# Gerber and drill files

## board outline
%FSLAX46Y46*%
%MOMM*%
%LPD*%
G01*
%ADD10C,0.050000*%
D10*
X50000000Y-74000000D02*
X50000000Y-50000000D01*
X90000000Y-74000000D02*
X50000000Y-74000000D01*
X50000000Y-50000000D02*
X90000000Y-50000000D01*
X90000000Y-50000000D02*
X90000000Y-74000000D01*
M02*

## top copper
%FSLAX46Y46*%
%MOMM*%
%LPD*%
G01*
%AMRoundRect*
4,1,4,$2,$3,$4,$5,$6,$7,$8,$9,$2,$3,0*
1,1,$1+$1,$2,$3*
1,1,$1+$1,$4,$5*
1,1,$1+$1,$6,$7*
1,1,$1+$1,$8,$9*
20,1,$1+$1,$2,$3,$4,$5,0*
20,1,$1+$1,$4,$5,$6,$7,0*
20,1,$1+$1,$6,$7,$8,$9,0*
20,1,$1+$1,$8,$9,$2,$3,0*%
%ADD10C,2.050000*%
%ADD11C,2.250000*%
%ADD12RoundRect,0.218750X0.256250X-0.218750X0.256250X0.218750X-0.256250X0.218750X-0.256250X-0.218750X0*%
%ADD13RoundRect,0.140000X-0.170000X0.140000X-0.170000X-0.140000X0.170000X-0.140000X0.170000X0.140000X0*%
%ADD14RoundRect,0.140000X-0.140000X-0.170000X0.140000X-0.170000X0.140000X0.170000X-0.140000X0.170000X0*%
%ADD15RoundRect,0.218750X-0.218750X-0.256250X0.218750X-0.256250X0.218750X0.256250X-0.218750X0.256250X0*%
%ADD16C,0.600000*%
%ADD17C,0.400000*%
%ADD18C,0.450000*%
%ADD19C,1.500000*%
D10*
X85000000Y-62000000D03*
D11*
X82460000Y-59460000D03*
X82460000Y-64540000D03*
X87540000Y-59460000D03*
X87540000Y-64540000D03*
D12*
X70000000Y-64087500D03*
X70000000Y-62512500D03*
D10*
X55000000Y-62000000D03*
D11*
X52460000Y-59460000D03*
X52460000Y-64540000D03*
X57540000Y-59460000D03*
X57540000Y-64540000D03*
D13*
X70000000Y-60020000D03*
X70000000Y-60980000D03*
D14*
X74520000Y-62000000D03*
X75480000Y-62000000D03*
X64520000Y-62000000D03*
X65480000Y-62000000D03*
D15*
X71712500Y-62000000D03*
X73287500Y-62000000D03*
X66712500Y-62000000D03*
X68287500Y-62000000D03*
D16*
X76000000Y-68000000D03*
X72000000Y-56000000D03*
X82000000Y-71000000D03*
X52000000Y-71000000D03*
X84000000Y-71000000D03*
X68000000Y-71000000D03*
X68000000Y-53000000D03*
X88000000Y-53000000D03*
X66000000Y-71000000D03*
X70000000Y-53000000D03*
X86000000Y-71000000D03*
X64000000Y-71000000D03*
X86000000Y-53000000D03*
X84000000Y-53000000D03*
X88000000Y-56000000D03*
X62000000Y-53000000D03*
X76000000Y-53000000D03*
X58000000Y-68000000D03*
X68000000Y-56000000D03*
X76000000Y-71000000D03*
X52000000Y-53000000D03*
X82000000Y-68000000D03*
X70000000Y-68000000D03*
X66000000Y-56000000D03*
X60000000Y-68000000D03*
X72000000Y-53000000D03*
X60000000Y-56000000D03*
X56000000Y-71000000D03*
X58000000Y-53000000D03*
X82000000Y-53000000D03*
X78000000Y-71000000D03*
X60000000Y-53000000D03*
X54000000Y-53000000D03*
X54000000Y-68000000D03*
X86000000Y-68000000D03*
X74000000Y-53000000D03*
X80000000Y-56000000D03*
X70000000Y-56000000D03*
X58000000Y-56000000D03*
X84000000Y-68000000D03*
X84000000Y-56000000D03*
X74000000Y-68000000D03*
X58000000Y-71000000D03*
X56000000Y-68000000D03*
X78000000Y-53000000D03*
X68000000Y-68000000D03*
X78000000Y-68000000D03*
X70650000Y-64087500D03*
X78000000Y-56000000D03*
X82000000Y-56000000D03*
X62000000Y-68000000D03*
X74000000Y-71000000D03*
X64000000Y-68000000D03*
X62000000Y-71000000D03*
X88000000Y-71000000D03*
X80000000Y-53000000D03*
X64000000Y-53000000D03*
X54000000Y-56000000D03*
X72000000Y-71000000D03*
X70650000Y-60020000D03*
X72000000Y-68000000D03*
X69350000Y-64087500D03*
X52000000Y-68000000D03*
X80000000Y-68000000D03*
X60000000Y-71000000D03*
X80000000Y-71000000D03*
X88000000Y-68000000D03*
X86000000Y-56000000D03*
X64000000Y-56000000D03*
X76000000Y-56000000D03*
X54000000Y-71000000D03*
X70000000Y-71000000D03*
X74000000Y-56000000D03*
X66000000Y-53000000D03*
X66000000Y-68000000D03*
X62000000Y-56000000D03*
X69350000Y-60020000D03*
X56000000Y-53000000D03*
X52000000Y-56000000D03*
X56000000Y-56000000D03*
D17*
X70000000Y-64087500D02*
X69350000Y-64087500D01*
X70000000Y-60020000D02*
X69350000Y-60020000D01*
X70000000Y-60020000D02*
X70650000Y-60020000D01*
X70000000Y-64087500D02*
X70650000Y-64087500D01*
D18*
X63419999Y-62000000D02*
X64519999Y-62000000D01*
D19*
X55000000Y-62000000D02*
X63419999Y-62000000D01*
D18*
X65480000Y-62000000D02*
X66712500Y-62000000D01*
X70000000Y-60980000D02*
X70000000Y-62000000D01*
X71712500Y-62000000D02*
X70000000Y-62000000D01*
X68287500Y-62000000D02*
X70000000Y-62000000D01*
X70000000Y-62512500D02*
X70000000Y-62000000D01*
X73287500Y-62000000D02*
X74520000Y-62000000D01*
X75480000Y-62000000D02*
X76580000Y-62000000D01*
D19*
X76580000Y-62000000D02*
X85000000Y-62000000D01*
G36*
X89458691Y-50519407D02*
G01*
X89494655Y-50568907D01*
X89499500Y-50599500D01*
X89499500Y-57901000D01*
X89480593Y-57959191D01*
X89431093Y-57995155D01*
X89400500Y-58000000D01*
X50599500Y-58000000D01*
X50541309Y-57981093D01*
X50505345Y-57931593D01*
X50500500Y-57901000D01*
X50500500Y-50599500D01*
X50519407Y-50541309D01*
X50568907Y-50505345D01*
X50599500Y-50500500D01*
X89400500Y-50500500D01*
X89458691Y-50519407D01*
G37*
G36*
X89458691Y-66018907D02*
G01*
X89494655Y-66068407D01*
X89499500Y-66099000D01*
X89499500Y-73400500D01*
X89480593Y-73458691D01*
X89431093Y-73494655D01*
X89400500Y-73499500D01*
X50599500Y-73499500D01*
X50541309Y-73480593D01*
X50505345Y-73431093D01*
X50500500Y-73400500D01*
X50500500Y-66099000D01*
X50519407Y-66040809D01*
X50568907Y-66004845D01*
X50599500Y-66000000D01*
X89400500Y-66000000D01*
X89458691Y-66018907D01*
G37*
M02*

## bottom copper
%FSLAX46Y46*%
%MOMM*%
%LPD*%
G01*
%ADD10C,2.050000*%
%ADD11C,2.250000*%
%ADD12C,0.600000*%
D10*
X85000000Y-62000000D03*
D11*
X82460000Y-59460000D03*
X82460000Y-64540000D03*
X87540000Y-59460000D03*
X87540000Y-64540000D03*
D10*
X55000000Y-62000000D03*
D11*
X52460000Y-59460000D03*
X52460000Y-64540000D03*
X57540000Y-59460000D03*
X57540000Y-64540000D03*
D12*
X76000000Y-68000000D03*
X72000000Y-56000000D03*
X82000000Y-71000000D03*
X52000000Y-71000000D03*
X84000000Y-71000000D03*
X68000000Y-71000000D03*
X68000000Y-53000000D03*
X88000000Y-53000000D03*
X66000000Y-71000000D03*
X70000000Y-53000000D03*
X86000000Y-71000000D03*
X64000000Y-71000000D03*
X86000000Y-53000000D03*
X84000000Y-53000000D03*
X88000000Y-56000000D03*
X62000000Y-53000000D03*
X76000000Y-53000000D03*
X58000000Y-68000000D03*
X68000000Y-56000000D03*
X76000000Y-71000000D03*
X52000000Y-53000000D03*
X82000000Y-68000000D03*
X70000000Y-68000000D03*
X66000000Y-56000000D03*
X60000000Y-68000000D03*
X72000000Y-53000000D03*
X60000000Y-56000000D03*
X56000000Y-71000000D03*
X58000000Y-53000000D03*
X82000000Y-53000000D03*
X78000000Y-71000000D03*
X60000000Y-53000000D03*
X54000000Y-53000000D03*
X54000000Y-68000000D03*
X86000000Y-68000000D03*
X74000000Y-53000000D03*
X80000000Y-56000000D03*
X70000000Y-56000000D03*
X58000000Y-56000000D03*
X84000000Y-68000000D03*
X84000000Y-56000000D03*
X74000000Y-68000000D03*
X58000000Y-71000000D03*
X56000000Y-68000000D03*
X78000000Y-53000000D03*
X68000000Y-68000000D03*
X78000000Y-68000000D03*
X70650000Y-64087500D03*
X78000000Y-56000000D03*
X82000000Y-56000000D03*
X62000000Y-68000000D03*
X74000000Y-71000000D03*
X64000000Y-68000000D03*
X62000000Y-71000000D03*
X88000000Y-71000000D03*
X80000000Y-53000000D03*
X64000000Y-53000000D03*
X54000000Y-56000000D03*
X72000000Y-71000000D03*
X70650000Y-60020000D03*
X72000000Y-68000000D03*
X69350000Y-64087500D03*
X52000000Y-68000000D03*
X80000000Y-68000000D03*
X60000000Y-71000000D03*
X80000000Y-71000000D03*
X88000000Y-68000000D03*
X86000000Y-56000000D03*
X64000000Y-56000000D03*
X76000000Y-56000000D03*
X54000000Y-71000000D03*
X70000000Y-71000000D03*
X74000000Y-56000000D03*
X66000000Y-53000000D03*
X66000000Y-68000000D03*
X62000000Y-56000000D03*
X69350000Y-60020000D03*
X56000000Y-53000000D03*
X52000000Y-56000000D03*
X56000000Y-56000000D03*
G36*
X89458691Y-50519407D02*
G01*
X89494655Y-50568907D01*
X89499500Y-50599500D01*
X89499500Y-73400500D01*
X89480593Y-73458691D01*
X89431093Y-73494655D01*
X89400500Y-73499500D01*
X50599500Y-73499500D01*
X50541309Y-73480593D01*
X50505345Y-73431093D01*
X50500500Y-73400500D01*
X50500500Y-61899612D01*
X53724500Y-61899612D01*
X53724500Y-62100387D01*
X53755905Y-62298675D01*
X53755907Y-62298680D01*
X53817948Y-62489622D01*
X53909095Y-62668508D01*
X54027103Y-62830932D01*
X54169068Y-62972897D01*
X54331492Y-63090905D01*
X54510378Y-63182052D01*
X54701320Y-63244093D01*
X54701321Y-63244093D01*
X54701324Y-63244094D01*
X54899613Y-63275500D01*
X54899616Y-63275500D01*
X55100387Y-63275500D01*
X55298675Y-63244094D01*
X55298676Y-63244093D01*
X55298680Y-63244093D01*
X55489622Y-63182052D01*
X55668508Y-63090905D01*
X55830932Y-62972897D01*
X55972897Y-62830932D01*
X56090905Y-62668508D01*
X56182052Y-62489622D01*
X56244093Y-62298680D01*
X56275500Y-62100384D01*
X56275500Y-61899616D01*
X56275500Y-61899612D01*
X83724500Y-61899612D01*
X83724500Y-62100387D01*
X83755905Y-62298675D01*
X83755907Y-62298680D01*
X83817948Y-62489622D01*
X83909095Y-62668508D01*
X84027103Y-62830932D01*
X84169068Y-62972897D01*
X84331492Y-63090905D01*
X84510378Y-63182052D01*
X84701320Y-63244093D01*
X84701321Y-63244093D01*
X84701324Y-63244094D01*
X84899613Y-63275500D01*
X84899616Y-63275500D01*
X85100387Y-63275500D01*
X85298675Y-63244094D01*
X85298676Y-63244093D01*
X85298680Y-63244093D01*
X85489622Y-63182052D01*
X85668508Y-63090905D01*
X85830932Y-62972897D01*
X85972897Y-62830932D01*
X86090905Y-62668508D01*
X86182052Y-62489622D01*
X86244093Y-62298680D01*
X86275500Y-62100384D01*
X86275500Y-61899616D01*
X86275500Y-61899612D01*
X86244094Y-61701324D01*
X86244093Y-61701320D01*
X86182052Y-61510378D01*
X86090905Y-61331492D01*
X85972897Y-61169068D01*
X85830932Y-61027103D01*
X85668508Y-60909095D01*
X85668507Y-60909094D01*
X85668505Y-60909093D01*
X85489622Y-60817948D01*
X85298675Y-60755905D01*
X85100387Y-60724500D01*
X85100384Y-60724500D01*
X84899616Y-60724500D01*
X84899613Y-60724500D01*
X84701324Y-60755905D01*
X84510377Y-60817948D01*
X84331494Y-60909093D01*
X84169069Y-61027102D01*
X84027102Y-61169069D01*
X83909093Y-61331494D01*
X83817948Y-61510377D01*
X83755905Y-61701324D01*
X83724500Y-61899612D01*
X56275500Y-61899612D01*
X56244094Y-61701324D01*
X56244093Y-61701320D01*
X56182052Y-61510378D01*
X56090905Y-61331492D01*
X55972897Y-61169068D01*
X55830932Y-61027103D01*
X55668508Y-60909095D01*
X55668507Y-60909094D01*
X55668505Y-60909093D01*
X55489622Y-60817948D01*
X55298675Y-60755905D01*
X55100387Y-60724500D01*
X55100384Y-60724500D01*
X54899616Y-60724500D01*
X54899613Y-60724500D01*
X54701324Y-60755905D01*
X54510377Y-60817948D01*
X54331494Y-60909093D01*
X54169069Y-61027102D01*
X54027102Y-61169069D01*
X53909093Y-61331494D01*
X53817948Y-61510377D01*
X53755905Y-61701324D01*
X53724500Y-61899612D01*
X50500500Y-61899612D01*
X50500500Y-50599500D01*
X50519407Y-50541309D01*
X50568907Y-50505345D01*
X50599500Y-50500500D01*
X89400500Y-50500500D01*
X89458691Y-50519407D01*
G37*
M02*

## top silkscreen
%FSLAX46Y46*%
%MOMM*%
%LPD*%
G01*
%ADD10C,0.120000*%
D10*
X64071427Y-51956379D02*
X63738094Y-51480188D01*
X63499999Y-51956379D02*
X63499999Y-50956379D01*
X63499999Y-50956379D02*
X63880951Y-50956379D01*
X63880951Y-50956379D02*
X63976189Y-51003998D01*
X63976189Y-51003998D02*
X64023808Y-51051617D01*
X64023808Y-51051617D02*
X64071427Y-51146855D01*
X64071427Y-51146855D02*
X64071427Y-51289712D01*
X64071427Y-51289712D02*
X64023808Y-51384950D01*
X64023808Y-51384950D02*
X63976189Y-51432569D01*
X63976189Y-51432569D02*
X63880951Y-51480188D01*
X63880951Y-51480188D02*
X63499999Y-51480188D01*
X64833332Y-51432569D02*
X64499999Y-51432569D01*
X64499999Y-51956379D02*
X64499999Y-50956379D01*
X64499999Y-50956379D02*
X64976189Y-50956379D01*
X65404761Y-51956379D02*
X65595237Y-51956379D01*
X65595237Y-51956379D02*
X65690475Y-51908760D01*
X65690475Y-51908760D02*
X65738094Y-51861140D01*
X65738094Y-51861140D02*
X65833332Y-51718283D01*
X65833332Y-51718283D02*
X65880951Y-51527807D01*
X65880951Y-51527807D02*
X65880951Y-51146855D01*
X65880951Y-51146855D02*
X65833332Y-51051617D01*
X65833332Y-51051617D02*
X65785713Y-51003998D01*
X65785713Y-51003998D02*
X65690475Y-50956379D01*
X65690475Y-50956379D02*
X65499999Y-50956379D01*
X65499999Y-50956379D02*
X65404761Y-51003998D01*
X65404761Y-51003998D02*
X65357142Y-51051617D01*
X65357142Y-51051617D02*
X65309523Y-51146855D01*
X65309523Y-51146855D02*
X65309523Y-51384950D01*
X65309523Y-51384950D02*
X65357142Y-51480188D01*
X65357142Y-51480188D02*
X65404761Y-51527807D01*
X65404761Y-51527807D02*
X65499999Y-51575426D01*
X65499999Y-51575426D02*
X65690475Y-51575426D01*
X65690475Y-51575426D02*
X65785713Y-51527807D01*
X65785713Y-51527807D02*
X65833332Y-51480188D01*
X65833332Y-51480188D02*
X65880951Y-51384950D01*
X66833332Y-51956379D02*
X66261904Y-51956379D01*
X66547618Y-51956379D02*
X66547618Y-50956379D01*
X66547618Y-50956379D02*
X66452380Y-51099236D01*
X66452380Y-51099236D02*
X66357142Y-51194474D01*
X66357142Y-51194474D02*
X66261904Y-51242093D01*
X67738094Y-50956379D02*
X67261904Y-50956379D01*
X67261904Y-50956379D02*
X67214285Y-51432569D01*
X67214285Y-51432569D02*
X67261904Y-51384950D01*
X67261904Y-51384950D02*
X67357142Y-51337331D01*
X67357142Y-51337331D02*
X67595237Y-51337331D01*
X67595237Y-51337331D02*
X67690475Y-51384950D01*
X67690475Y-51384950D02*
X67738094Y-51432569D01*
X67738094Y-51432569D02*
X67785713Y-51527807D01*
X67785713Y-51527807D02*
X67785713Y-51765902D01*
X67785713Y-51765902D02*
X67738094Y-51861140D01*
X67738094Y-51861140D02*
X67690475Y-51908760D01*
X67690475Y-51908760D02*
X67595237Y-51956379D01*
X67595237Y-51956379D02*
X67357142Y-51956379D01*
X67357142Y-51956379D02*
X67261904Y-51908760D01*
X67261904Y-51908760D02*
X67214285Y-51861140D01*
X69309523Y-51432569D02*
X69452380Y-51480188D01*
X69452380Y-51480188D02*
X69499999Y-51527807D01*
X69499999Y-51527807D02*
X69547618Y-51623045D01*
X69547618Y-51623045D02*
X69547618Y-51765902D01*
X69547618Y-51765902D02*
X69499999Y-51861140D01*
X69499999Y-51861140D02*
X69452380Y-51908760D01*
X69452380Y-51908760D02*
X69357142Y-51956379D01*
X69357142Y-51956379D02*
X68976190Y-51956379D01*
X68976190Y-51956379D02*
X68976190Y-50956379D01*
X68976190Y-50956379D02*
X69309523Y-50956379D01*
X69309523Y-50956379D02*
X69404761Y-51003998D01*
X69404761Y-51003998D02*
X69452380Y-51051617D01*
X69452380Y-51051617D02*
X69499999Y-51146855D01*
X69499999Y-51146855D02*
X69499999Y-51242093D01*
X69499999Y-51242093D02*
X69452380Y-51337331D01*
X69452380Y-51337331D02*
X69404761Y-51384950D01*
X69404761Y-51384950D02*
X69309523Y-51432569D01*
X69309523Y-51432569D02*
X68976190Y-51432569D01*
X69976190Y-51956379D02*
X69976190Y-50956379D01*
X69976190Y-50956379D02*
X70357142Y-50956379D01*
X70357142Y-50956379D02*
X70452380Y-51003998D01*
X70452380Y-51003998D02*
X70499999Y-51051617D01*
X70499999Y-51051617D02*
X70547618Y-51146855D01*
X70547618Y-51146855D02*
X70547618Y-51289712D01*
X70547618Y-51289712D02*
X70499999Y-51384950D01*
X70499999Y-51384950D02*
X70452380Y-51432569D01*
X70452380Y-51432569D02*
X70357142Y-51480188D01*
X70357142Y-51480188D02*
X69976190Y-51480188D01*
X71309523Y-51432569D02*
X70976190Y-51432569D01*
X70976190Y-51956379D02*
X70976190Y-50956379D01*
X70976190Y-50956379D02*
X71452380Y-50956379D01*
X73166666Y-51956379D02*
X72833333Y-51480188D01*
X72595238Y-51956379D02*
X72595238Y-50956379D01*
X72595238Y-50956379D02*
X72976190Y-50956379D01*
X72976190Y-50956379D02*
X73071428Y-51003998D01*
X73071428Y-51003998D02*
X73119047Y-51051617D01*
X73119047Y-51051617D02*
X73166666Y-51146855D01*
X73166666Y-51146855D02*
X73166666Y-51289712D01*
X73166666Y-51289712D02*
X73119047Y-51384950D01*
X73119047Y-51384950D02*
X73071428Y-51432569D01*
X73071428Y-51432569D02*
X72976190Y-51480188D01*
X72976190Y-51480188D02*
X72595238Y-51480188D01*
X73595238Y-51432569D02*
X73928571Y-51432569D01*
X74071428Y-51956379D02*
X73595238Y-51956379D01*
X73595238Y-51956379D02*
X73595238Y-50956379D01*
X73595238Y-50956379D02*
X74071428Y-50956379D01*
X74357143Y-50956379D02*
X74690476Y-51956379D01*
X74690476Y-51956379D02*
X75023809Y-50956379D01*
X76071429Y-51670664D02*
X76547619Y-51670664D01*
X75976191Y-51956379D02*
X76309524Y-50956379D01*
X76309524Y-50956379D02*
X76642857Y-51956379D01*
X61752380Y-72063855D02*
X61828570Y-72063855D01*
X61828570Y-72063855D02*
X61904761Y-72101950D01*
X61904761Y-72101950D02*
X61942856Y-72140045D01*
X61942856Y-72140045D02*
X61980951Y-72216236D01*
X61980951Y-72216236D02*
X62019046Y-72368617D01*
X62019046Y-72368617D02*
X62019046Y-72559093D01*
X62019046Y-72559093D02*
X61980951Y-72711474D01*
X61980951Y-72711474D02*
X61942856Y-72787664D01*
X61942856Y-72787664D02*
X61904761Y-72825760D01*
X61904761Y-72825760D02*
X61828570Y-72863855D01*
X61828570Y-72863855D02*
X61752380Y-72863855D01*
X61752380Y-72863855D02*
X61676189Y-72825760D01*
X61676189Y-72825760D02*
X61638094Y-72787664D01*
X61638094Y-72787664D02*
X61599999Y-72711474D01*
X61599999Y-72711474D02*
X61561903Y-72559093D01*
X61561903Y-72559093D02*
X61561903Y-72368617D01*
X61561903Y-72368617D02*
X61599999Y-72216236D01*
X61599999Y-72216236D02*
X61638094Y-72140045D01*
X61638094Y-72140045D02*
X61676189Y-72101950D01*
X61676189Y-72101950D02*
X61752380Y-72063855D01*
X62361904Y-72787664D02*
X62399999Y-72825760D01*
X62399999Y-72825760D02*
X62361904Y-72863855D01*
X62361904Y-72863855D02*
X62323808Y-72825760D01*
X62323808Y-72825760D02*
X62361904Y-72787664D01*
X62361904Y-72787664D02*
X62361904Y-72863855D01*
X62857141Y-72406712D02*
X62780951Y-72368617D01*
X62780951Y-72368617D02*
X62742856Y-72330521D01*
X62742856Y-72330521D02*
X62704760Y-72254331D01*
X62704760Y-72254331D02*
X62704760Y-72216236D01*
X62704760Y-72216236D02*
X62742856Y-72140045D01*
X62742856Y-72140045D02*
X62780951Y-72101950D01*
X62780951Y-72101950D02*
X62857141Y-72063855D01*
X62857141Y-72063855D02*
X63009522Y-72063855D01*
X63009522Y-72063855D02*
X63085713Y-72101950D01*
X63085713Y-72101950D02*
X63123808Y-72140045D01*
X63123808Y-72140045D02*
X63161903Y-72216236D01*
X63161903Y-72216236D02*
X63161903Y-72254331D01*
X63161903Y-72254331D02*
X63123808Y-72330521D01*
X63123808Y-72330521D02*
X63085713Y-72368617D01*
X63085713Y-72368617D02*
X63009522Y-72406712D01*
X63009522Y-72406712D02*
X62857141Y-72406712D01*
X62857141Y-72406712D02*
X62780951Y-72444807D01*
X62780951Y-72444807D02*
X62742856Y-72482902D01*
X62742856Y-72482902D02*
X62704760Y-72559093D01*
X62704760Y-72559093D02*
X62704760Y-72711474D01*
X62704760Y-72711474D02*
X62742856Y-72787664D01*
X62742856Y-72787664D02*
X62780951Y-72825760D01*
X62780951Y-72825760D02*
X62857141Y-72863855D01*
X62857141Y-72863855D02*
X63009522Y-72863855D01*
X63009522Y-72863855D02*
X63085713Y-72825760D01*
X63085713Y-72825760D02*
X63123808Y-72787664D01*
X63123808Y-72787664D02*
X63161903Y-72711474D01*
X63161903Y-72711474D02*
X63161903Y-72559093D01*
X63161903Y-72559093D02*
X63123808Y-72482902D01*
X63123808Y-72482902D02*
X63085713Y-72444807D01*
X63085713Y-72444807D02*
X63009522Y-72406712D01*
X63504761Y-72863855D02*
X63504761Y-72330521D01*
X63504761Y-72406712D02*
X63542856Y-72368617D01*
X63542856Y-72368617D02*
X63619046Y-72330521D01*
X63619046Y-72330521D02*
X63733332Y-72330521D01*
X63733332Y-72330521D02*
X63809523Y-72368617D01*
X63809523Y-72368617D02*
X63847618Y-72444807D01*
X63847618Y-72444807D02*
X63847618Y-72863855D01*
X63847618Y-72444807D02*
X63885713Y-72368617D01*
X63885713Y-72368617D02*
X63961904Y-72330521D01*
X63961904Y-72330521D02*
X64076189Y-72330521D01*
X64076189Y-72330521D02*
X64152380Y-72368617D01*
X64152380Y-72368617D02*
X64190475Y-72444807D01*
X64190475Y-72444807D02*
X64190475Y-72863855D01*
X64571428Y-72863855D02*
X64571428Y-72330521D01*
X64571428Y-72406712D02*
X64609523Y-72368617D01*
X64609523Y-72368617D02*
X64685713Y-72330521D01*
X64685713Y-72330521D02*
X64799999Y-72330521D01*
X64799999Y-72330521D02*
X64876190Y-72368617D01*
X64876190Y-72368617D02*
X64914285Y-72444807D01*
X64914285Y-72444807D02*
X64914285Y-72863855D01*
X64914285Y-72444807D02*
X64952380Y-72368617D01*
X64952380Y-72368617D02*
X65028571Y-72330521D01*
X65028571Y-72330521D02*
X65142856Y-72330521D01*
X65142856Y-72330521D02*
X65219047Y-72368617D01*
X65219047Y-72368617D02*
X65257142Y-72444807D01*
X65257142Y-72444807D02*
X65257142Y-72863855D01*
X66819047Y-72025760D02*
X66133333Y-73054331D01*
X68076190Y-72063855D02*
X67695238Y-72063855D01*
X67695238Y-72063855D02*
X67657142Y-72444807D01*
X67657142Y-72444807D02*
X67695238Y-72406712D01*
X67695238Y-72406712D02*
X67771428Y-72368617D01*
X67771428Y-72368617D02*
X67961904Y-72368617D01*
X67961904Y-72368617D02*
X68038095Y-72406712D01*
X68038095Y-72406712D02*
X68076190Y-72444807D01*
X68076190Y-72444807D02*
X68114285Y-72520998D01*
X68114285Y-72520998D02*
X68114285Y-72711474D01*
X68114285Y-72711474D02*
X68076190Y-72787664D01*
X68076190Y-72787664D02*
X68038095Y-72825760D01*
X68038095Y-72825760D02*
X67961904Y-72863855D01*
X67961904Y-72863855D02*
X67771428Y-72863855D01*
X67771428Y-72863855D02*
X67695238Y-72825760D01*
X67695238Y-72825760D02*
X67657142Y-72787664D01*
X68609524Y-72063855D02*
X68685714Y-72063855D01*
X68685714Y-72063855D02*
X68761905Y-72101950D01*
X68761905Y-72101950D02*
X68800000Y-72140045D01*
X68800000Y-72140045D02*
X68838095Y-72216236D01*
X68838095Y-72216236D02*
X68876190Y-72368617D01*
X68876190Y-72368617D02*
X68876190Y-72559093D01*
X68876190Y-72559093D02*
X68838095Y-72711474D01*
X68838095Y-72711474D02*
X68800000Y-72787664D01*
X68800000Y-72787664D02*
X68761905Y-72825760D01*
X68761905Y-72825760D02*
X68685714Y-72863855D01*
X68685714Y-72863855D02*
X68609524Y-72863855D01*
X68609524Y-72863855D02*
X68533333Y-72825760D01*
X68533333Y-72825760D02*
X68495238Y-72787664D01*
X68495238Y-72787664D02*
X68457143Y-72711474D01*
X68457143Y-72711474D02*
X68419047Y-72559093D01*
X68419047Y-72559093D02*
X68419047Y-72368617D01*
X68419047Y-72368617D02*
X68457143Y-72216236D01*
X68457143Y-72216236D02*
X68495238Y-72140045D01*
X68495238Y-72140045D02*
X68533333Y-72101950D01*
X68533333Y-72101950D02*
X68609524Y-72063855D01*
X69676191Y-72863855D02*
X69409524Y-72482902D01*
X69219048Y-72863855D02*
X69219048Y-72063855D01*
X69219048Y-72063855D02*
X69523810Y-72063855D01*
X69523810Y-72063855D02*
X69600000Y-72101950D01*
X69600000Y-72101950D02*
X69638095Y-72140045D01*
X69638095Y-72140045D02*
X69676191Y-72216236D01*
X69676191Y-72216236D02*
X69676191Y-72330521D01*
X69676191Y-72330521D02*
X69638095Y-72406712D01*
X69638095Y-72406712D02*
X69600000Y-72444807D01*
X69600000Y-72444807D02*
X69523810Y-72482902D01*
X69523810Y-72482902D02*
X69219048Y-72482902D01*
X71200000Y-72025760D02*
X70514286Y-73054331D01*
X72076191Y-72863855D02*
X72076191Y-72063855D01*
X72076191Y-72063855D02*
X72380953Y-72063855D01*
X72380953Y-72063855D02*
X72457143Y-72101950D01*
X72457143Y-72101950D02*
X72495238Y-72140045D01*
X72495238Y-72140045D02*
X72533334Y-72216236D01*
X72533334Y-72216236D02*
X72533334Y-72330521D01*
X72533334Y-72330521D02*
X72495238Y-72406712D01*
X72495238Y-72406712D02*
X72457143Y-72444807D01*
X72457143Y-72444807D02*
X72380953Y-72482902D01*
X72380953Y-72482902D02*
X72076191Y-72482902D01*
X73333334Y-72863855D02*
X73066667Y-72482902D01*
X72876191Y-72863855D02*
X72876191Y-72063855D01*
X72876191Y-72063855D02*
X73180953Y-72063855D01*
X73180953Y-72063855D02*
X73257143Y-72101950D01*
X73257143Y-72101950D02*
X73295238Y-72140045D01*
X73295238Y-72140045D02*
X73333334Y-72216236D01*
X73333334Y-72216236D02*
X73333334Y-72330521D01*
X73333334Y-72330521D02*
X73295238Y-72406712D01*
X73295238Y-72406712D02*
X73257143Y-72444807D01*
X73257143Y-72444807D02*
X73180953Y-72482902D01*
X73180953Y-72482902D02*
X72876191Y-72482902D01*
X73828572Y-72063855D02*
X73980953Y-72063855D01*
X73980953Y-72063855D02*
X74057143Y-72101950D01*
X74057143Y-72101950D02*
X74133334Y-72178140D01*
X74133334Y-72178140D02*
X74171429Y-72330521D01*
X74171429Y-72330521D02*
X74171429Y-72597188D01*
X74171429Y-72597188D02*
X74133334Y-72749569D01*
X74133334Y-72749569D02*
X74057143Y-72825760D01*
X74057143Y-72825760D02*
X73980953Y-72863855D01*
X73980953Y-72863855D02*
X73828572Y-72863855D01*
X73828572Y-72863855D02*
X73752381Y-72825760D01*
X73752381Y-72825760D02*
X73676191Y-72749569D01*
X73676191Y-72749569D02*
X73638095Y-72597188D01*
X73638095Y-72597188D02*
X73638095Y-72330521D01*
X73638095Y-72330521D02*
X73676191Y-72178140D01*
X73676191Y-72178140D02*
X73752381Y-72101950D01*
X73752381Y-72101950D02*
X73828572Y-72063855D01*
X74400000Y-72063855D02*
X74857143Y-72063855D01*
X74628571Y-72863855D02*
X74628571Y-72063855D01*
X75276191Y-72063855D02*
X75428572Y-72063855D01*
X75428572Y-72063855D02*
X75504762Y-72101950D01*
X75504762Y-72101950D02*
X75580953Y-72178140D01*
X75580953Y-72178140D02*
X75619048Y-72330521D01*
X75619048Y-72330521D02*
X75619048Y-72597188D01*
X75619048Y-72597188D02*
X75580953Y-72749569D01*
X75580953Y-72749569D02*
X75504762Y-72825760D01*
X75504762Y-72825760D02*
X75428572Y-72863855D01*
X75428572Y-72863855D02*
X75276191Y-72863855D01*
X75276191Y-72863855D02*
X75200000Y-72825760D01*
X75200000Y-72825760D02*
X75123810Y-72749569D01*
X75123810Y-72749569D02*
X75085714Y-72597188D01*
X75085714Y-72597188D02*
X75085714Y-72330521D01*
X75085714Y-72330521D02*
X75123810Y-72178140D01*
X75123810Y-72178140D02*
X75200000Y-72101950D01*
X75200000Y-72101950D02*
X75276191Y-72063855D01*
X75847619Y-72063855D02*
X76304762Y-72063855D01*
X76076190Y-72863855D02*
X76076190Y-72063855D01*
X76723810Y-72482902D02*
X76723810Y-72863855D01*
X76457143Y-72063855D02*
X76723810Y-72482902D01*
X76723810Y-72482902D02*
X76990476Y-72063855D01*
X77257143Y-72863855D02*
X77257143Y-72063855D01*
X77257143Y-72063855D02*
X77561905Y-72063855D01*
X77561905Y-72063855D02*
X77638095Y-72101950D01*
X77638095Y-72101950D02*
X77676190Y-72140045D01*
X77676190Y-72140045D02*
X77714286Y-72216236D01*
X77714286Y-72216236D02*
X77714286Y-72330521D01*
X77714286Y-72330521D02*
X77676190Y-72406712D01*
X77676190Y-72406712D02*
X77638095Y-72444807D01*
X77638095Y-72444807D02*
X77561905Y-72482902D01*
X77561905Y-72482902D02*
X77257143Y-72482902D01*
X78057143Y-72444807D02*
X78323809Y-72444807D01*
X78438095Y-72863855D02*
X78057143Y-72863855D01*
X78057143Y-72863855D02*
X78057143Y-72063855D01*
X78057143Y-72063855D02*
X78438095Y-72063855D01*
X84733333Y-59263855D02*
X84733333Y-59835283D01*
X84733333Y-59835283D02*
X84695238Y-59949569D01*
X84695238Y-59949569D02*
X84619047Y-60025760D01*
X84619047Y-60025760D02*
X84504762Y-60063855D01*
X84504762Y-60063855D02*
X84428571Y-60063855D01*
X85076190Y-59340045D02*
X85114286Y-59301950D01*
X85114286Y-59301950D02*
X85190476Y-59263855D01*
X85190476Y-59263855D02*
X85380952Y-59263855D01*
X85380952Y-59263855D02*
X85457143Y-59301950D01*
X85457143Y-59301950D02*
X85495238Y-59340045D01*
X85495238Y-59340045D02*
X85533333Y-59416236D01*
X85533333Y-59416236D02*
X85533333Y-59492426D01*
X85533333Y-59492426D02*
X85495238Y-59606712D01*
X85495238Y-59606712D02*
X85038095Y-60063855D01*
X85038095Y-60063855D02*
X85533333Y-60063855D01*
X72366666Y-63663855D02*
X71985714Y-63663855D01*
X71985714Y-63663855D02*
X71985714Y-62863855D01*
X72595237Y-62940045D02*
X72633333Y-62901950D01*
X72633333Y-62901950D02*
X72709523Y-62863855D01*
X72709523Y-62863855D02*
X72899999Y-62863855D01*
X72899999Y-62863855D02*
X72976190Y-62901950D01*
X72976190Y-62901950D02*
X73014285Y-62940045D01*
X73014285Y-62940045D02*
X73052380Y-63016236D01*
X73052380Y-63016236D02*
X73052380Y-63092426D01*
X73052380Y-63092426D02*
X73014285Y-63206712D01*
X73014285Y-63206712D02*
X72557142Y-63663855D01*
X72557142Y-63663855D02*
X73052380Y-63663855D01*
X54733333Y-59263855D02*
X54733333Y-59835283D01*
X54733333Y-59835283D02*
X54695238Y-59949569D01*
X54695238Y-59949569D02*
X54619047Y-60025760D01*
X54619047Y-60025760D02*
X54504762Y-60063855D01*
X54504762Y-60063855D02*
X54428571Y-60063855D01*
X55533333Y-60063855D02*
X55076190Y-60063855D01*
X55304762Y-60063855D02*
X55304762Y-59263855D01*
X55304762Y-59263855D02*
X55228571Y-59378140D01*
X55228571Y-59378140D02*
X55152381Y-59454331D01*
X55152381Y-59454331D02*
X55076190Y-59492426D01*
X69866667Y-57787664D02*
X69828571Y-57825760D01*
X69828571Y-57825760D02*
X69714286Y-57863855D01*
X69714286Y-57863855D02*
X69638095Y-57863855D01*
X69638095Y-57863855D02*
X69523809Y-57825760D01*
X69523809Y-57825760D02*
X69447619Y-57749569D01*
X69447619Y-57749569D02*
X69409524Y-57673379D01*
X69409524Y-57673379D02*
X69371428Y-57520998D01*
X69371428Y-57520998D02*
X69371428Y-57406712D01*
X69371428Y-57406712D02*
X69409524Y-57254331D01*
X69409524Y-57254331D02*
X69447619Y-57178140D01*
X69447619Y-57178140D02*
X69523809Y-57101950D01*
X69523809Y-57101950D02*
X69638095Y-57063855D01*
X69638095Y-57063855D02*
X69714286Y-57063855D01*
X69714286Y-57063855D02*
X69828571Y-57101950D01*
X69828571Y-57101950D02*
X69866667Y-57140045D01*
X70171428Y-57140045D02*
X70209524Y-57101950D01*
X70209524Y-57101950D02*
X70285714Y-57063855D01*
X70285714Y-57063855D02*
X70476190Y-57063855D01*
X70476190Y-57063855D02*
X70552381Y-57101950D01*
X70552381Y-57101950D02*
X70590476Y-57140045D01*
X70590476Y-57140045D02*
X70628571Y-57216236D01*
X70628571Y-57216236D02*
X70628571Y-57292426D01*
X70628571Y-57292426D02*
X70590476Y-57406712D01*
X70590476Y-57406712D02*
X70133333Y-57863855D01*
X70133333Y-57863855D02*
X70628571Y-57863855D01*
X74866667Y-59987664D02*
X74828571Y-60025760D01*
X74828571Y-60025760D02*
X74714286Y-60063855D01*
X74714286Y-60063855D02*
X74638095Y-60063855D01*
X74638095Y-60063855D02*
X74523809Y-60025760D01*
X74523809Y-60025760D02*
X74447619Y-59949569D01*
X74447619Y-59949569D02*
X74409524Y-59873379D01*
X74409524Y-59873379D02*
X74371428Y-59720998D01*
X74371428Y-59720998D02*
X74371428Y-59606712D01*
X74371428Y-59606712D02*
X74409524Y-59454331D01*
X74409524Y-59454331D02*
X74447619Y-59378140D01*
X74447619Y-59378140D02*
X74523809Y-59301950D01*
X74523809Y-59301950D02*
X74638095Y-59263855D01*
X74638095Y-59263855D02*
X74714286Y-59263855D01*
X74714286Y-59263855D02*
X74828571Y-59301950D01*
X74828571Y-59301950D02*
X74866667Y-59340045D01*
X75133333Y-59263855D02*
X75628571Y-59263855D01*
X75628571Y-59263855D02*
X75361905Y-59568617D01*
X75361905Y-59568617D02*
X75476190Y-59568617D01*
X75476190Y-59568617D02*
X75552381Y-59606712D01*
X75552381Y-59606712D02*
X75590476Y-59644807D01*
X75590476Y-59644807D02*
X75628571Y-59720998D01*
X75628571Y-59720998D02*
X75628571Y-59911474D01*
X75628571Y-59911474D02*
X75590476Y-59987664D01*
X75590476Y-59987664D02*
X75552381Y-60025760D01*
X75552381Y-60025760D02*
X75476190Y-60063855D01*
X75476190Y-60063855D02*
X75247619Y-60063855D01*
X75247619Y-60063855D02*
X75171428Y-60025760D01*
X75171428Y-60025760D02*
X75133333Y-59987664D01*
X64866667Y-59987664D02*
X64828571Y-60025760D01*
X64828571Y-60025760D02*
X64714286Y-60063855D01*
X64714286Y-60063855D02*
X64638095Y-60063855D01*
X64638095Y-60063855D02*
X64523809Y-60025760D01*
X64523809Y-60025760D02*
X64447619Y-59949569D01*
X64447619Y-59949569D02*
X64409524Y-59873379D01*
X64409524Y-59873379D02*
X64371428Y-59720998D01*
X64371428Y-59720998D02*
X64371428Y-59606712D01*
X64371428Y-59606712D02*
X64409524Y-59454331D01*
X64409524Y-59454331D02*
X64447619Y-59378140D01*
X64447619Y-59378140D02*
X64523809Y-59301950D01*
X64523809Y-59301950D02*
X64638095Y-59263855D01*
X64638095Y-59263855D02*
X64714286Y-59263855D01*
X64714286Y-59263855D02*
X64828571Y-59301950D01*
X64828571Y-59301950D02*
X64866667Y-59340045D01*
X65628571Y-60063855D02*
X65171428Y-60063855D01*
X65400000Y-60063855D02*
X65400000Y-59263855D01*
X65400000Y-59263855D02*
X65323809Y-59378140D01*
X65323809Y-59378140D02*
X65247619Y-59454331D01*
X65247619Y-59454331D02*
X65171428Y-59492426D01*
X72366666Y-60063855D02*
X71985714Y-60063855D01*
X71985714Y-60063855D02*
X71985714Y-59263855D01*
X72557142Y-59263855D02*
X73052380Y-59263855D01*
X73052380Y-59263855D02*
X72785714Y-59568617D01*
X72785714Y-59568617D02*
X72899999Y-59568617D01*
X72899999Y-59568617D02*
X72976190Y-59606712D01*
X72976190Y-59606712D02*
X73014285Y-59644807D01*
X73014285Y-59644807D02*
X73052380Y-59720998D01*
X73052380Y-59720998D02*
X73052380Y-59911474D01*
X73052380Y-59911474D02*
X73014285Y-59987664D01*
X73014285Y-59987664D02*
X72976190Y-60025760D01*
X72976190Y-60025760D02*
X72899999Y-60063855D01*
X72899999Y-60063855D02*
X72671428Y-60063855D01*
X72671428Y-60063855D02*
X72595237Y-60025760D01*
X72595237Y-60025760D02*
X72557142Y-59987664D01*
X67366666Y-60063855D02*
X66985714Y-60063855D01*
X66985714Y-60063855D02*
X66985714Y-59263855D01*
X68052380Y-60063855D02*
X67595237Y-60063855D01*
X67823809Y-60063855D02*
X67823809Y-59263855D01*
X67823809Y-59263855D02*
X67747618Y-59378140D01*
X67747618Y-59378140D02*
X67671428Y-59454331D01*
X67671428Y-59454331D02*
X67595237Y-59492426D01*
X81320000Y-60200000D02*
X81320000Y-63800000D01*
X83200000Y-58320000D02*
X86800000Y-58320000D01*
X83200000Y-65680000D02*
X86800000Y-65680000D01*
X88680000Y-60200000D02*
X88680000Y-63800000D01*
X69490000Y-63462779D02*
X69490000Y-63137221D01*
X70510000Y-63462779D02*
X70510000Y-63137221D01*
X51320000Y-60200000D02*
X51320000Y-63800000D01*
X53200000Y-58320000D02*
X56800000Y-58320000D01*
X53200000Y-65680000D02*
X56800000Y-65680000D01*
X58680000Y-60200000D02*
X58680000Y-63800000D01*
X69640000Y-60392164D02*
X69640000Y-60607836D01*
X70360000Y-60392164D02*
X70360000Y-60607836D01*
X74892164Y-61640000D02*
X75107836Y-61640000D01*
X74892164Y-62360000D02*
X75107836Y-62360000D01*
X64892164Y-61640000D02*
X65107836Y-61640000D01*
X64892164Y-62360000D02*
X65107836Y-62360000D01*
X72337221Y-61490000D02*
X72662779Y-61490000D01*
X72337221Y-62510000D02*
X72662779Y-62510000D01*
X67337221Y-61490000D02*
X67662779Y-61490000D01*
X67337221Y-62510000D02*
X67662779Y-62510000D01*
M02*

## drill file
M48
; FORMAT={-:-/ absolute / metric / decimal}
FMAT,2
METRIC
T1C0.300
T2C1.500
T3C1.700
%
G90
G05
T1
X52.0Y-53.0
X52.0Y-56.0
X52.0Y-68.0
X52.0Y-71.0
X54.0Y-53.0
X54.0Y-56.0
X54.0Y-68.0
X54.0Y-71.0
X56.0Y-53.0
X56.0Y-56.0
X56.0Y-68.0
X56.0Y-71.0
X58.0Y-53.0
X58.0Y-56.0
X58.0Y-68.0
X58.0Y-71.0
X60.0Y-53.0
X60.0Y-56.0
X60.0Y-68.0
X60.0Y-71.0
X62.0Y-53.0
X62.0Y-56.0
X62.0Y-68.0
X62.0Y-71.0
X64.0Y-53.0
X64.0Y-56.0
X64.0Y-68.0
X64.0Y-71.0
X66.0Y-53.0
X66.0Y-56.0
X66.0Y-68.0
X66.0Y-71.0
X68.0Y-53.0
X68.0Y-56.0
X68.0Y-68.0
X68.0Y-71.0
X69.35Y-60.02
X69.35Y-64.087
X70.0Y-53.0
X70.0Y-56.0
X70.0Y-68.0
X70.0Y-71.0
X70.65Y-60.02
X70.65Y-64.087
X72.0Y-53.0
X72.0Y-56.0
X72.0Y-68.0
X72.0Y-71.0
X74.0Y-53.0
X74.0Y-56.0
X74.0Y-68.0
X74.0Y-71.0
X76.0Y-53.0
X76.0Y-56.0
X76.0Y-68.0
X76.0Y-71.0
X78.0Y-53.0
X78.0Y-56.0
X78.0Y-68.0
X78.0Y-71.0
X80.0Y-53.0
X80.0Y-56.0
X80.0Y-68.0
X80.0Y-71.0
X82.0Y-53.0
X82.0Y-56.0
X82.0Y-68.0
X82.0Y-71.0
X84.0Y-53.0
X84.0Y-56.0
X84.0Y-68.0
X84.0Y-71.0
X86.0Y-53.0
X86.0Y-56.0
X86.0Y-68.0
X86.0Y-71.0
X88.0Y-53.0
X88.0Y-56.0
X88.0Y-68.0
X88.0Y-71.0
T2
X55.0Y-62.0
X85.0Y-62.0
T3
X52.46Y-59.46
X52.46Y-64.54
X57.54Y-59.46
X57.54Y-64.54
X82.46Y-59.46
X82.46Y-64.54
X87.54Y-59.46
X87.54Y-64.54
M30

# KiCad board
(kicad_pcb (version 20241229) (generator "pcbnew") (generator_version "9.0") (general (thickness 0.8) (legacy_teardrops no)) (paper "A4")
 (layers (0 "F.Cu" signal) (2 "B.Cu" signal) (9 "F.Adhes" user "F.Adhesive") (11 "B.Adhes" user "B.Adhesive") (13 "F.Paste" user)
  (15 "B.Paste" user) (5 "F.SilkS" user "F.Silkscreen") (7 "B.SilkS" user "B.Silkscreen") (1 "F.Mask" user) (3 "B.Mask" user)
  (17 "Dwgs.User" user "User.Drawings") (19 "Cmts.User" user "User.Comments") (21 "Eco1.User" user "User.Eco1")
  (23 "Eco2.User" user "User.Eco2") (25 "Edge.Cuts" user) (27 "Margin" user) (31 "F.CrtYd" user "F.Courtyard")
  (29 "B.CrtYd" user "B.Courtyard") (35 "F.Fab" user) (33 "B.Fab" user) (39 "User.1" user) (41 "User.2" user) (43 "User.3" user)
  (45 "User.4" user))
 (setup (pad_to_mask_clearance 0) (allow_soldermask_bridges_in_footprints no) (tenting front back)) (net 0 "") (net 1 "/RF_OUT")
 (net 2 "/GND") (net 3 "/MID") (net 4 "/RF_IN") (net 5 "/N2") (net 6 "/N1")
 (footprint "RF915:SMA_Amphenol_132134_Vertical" (layer "F.Cu") (at 85 62)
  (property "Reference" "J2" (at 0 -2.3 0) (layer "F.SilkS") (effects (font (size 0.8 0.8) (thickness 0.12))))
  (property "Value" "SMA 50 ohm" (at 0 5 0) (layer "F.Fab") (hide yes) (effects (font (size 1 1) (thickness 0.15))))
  (fp_line (start -3.68 -1.8) (end -3.68 1.8) (stroke (width 0.12) (type solid)) (layer "F.SilkS"))
  (fp_line (start -1.8 -3.68) (end 1.8 -3.68) (stroke (width 0.12) (type solid)) (layer "F.SilkS"))
  (fp_line (start -1.8 3.68) (end 1.8 3.68) (stroke (width 0.12) (type solid)) (layer "F.SilkS"))
  (fp_line (start 3.68 -1.8) (end 3.68 1.8) (stroke (width 0.12) (type solid)) (layer "F.SilkS"))
  (pad "1" thru_hole circle (at 0 0) (size 2.05 2.05) (drill 1.5) (layers "*.Cu" "*.Mask") (remove_unused_layers no) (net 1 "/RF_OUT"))
  (pad "2" thru_hole circle (at -2.54 -2.54) (size 2.25 2.25) (drill 1.7) (layers "*.Cu" "*.Mask") (remove_unused_layers no) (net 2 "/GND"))
  (pad "2" thru_hole circle (at -2.54 2.54) (size 2.25 2.25) (drill 1.7) (layers "*.Cu" "*.Mask") (remove_unused_layers no) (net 2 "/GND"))
  (pad "2" thru_hole circle (at 2.54 -2.54) (size 2.25 2.25) (drill 1.7) (layers "*.Cu" "*.Mask") (remove_unused_layers no) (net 2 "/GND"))
  (pad "2" thru_hole circle (at 2.54 2.54) (size 2.25 2.25) (drill 1.7) (layers "*.Cu" "*.Mask") (remove_unused_layers no) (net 2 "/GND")))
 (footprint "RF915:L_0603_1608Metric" (layer "F.Cu") (at 70 63.3 90)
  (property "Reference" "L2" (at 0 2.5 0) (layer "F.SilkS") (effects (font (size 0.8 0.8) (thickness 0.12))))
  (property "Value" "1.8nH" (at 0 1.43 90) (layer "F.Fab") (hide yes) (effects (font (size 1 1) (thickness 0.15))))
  (fp_line (start -0.162779 -0.51) (end 0.162779 -0.51) (stroke (width 0.12) (type solid)) (layer "F.SilkS"))
  (fp_line (start -0.162779 0.51) (end 0.162779 0.51) (stroke (width 0.12) (type solid)) (layer "F.SilkS"))
  (pad "1" smd roundrect (at -0.7875 0 90) (size 0.875 0.95) (layers "F.Cu" "F.Mask" "F.Paste") (roundrect_rratio 0.25) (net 2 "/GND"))
  (pad "2" smd roundrect (at 0.7875 0 90) (size 0.875 0.95) (layers "F.Cu" "F.Mask" "F.Paste") (roundrect_rratio 0.25) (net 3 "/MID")))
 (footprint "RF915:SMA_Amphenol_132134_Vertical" (layer "F.Cu") (at 55 62)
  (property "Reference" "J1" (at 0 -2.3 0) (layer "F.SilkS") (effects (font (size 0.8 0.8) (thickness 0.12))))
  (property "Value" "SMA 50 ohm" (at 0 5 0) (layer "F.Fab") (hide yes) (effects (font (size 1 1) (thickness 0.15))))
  (fp_line (start -3.68 -1.8) (end -3.68 1.8) (stroke (width 0.12) (type solid)) (layer "F.SilkS"))
  (fp_line (start -1.8 -3.68) (end 1.8 -3.68) (stroke (width 0.12) (type solid)) (layer "F.SilkS"))
  (fp_line (start -1.8 3.68) (end 1.8 3.68) (stroke (width 0.12) (type solid)) (layer "F.SilkS"))
  (fp_line (start 3.68 -1.8) (end 3.68 1.8) (stroke (width 0.12) (type solid)) (layer "F.SilkS"))
  (pad "1" thru_hole circle (at 0 0) (size 2.05 2.05) (drill 1.5) (layers "*.Cu" "*.Mask") (remove_unused_layers no) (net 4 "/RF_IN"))
  (pad "2" thru_hole circle (at -2.54 -2.54) (size 2.25 2.25) (drill 1.7) (layers "*.Cu" "*.Mask") (remove_unused_layers no) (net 2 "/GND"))
  (pad "2" thru_hole circle (at -2.54 2.54) (size 2.25 2.25) (drill 1.7) (layers "*.Cu" "*.Mask") (remove_unused_layers no) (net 2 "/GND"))
  (pad "2" thru_hole circle (at 2.54 -2.54) (size 2.25 2.25) (drill 1.7) (layers "*.Cu" "*.Mask") (remove_unused_layers no) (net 2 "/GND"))
  (pad "2" thru_hole circle (at 2.54 2.54) (size 2.25 2.25) (drill 1.7) (layers "*.Cu" "*.Mask") (remove_unused_layers no) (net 2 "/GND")))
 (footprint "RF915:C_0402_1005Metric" (layer "F.Cu") (at 70 60.5 -90)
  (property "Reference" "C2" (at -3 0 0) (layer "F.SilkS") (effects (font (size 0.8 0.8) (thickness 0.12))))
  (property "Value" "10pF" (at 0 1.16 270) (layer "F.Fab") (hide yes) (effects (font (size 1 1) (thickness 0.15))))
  (fp_line (start -0.107836 0.36) (end 0.107836 0.36) (stroke (width 0.12) (type solid)) (layer "F.SilkS"))
  (fp_line (start -0.107836 -0.36) (end 0.107836 -0.36) (stroke (width 0.12) (type solid)) (layer "F.SilkS"))
  (pad "1" smd roundrect (at -0.48 0 270) (size 0.56 0.62) (layers "F.Cu" "F.Mask" "F.Paste") (roundrect_rratio 0.25) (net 2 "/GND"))
  (pad "2" smd roundrect (at 0.48 0 270) (size 0.56 0.62) (layers "F.Cu" "F.Mask" "F.Paste") (roundrect_rratio 0.25) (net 3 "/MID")))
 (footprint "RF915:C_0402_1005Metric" (layer "F.Cu") (at 75 62)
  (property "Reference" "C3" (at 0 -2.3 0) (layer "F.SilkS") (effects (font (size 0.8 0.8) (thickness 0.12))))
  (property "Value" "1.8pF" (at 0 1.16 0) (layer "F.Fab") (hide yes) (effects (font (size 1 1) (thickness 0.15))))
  (fp_line (start -0.107836 -0.36) (end 0.107836 -0.36) (stroke (width 0.12) (type solid)) (layer "F.SilkS"))
  (fp_line (start -0.107836 0.36) (end 0.107836 0.36) (stroke (width 0.12) (type solid)) (layer "F.SilkS"))
  (pad "1" smd roundrect (at -0.48 0) (size 0.56 0.62) (layers "F.Cu" "F.Mask" "F.Paste") (roundrect_rratio 0.25) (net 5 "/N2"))
  (pad "2" smd roundrect (at 0.48 0) (size 0.56 0.62) (layers "F.Cu" "F.Mask" "F.Paste") (roundrect_rratio 0.25) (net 1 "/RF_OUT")))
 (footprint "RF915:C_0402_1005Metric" (layer "F.Cu") (at 65 62)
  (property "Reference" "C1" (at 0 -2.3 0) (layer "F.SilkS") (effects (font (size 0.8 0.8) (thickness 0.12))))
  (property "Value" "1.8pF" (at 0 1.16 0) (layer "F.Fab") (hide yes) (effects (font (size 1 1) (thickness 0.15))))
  (fp_line (start -0.107836 -0.36) (end 0.107836 -0.36) (stroke (width 0.12) (type solid)) (layer "F.SilkS"))
  (fp_line (start -0.107836 0.36) (end 0.107836 0.36) (stroke (width 0.12) (type solid)) (layer "F.SilkS"))
  (pad "1" smd roundrect (at -0.48 0) (size 0.56 0.62) (layers "F.Cu" "F.Mask" "F.Paste") (roundrect_rratio 0.25) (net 4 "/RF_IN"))
  (pad "2" smd roundrect (at 0.48 0) (size 0.56 0.62) (layers "F.Cu" "F.Mask" "F.Paste") (roundrect_rratio 0.25) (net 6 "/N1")))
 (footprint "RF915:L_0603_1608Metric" (layer "F.Cu") (at 72.5 62)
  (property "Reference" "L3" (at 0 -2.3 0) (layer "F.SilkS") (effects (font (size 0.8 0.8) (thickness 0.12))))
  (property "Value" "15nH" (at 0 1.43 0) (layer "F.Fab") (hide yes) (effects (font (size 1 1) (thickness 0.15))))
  (fp_line (start -0.162779 -0.51) (end 0.162779 -0.51) (stroke (width 0.12) (type solid)) (layer "F.SilkS"))
  (fp_line (start -0.162779 0.51) (end 0.162779 0.51) (stroke (width 0.12) (type solid)) (layer "F.SilkS"))
  (pad "1" smd roundrect (at -0.7875 0) (size 0.875 0.95) (layers "F.Cu" "F.Mask" "F.Paste") (roundrect_rratio 0.25) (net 3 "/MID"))
  (pad "2" smd roundrect (at 0.7875 0) (size 0.875 0.95) (layers "F.Cu" "F.Mask" "F.Paste") (roundrect_rratio 0.25) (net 5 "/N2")))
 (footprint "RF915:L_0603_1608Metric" (layer "F.Cu") (at 67.5 62)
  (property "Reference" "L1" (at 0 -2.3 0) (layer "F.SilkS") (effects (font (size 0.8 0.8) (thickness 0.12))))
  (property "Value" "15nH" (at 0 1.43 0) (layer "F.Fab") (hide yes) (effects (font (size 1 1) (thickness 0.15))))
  (fp_line (start -0.162779 -0.51) (end 0.162779 -0.51) (stroke (width 0.12) (type solid)) (layer "F.SilkS"))
  (fp_line (start -0.162779 0.51) (end 0.162779 0.51) (stroke (width 0.12) (type solid)) (layer "F.SilkS"))
  (pad "1" smd roundrect (at -0.7875 0) (size 0.875 0.95) (layers "F.Cu" "F.Mask" "F.Paste") (roundrect_rratio 0.25) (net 6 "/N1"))
  (pad "2" smd roundrect (at 0.7875 0) (size 0.875 0.95) (layers "F.Cu" "F.Mask" "F.Paste") (roundrect_rratio 0.25) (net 3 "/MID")))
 (gr_line (start 50 74) (end 50 50) (stroke (width 0.05) (type default)) (layer "Edge.Cuts"))
 (gr_line (start 90 74) (end 50 74) (stroke (width 0.05) (type default)) (layer "Edge.Cuts"))
 (gr_line (start 50 50) (end 90 50) (stroke (width 0.05) (type default)) (layer "Edge.Cuts"))
 (gr_line (start 90 50) (end 90 74) (stroke (width 0.05) (type default)) (layer "Edge.Cuts"))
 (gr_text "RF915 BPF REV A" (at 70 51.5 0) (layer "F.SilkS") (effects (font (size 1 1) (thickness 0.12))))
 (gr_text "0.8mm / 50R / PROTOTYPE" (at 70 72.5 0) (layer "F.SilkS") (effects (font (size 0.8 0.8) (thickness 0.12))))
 (segment (start 70 64.0875) (end 69.35 64.0875) (width 0.4) (layer "F.Cu") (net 2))
 (segment (start 70 60.02) (end 69.35 60.02) (width 0.4) (layer "F.Cu") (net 2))
 (segment (start 70 60.02) (end 70.65 60.02) (width 0.4) (layer "F.Cu") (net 2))
 (segment (start 70 64.0875) (end 70.65 64.0875) (width 0.4) (layer "F.Cu") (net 2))
 (via (at 76 68) (size 0.6) (drill 0.3) (layers "F.Cu" "B.Cu") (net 2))
 (via (at 72 56) (size 0.6) (drill 0.3) (layers "F.Cu" "B.Cu") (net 2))
 (via (at 82 71) (size 0.6) (drill 0.3) (layers "F.Cu" "B.Cu") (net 2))
 (via (at 52 71) (size 0.6) (drill 0.3) (layers "F.Cu" "B.Cu") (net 2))
 (via (at 84 71) (size 0.6) (drill 0.3) (layers "F.Cu" "B.Cu") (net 2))
 (via (at 68 71) (size 0.6) (drill 0.3) (layers "F.Cu" "B.Cu") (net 2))
 (via (at 68 53) (size 0.6) (drill 0.3) (layers "F.Cu" "B.Cu") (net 2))
 (via (at 88 53) (size 0.6) (drill 0.3) (layers "F.Cu" "B.Cu") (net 2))
 (via (at 66 71) (size 0.6) (drill 0.3) (layers "F.Cu" "B.Cu") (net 2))
 (via (at 70 53) (size 0.6) (drill 0.3) (layers "F.Cu" "B.Cu") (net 2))
 (via (at 86 71) (size 0.6) (drill 0.3) (layers "F.Cu" "B.Cu") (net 2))
 (via (at 64 71) (size 0.6) (drill 0.3) (layers "F.Cu" "B.Cu") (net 2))
 (via (at 86 53) (size 0.6) (drill 0.3) (layers "F.Cu" "B.Cu") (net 2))
 (via (at 84 53) (size 0.6) (drill 0.3) (layers "F.Cu" "B.Cu") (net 2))
 (via (at 88 56) (size 0.6) (drill 0.3) (layers "F.Cu" "B.Cu") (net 2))
 (via (at 62 53) (size 0.6) (drill 0.3) (layers "F.Cu" "B.Cu") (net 2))
 (via (at 76 53) (size 0.6) (drill 0.3) (layers "F.Cu" "B.Cu") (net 2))
 (via (at 58 68) (size 0.6) (drill 0.3) (layers "F.Cu" "B.Cu") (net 2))
 (via (at 68 56) (size 0.6) (drill 0.3) (layers "F.Cu" "B.Cu") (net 2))
 (via (at 76 71) (size 0.6) (drill 0.3) (layers "F.Cu" "B.Cu") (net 2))
 (via (at 52 53) (size 0.6) (drill 0.3) (layers "F.Cu" "B.Cu") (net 2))
 (via (at 82 68) (size 0.6) (drill 0.3) (layers "F.Cu" "B.Cu") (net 2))
 (via (at 70 68) (size 0.6) (drill 0.3) (layers "F.Cu" "B.Cu") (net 2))
 (via (at 66 56) (size 0.6) (drill 0.3) (layers "F.Cu" "B.Cu") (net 2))
 (via (at 60 68) (size 0.6) (drill 0.3) (layers "F.Cu" "B.Cu") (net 2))
 (via (at 72 53) (size 0.6) (drill 0.3) (layers "F.Cu" "B.Cu") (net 2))
 (via (at 60 56) (size 0.6) (drill 0.3) (layers "F.Cu" "B.Cu") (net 2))
 (via (at 56 71) (size 0.6) (drill 0.3) (layers "F.Cu" "B.Cu") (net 2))
 (via (at 58 53) (size 0.6) (drill 0.3) (layers "F.Cu" "B.Cu") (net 2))
 (via (at 82 53) (size 0.6) (drill 0.3) (layers "F.Cu" "B.Cu") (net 2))
 (via (at 78 71) (size 0.6) (drill 0.3) (layers "F.Cu" "B.Cu") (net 2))
 (via (at 60 53) (size 0.6) (drill 0.3) (layers "F.Cu" "B.Cu") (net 2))
 (via (at 54 53) (size 0.6) (drill 0.3) (layers "F.Cu" "B.Cu") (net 2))
 (via (at 54 68) (size 0.6) (drill 0.3) (layers "F.Cu" "B.Cu") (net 2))
 (via (at 86 68) (size 0.6) (drill 0.3) (layers "F.Cu" "B.Cu") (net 2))
 (via (at 74 53) (size 0.6) (drill 0.3) (layers "F.Cu" "B.Cu") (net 2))
 (via (at 80 56) (size 0.6) (drill 0.3) (layers "F.Cu" "B.Cu") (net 2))
 (via (at 70 56) (size 0.6) (drill 0.3) (layers "F.Cu" "B.Cu") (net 2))
 (via (at 58 56) (size 0.6) (drill 0.3) (layers "F.Cu" "B.Cu") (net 2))
 (via (at 84 68) (size 0.6) (drill 0.3) (layers "F.Cu" "B.Cu") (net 2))
 (via (at 84 56) (size 0.6) (drill 0.3) (layers "F.Cu" "B.Cu") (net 2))
 (via (at 74 68) (size 0.6) (drill 0.3) (layers "F.Cu" "B.Cu") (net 2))
 (via (at 58 71) (size 0.6) (drill 0.3) (layers "F.Cu" "B.Cu") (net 2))
 (via (at 56 68) (size 0.6) (drill 0.3) (layers "F.Cu" "B.Cu") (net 2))
 (via (at 78 53) (size 0.6) (drill 0.3) (layers "F.Cu" "B.Cu") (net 2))
 (via (at 68 68) (size 0.6) (drill 0.3) (layers "F.Cu" "B.Cu") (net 2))
 (via (at 78 68) (size 0.6) (drill 0.3) (layers "F.Cu" "B.Cu") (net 2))
 (via (at 70.65 64.0875) (size 0.6) (drill 0.3) (layers "F.Cu" "B.Cu") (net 2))
 (via (at 78 56) (size 0.6) (drill 0.3) (layers "F.Cu" "B.Cu") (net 2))
 (via (at 82 56) (size 0.6) (drill 0.3) (layers "F.Cu" "B.Cu") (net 2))
 (via (at 62 68) (size 0.6) (drill 0.3) (layers "F.Cu" "B.Cu") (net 2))
 (via (at 74 71) (size 0.6) (drill 0.3) (layers "F.Cu" "B.Cu") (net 2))
 (via (at 64 68) (size 0.6) (drill 0.3) (layers "F.Cu" "B.Cu") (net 2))
 (via (at 62 71) (size 0.6) (drill 0.3) (layers "F.Cu" "B.Cu") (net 2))
 (via (at 88 71) (size 0.6) (drill 0.3) (layers "F.Cu" "B.Cu") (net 2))
 (via (at 80 53) (size 0.6) (drill 0.3) (layers "F.Cu" "B.Cu") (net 2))
 (via (at 64 53) (size 0.6) (drill 0.3) (layers "F.Cu" "B.Cu") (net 2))
 (via (at 54 56) (size 0.6) (drill 0.3) (layers "F.Cu" "B.Cu") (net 2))
 (via (at 72 71) (size 0.6) (drill 0.3) (layers "F.Cu" "B.Cu") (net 2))
 (via (at 70.65 60.02) (size 0.6) (drill 0.3) (layers "F.Cu" "B.Cu") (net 2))
 (via (at 72 68) (size 0.6) (drill 0.3) (layers "F.Cu" "B.Cu") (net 2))
 (via (at 69.35 64.0875) (size 0.6) (drill 0.3) (layers "F.Cu" "B.Cu") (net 2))
 (via (at 52 68) (size 0.6) (drill 0.3) (layers "F.Cu" "B.Cu") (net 2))
 (via (at 80 68) (size 0.6) (drill 0.3) (layers "F.Cu" "B.Cu") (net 2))
 (via (at 60 71) (size 0.6) (drill 0.3) (layers "F.Cu" "B.Cu") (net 2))
 (via (at 80 71) (size 0.6) (drill 0.3) (layers "F.Cu" "B.Cu") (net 2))
 (via (at 88 68) (size 0.6) (drill 0.3) (layers "F.Cu" "B.Cu") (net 2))
 (via (at 86 56) (size 0.6) (drill 0.3) (layers "F.Cu" "B.Cu") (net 2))
 (via (at 64 56) (size 0.6) (drill 0.3) (layers "F.Cu" "B.Cu") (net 2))
 (via (at 76 56) (size 0.6) (drill 0.3) (layers "F.Cu" "B.Cu") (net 2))
 (via (at 54 71) (size 0.6) (drill 0.3) (layers "F.Cu" "B.Cu") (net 2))
 (via (at 70 71) (size 0.6) (drill 0.3) (layers "F.Cu" "B.Cu") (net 2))
 (via (at 74 56) (size 0.6) (drill 0.3) (layers "F.Cu" "B.Cu") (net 2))
 (via (at 66 53) (size 0.6) (drill 0.3) (layers "F.Cu" "B.Cu") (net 2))
 (via (at 66 68) (size 0.6) (drill 0.3) (layers "F.Cu" "B.Cu") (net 2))
 (via (at 62 56) (size 0.6) (drill 0.3) (layers "F.Cu" "B.Cu") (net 2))
 (via (at 69.35 60.02) (size 0.6) (drill 0.3) (layers "F.Cu" "B.Cu") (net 2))
 (via (at 56 53) (size 0.6) (drill 0.3) (layers "F.Cu" "B.Cu") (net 2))
 (via (at 52 56) (size 0.6) (drill 0.3) (layers "F.Cu" "B.Cu") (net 2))
 (via (at 56 56) (size 0.6) (drill 0.3) (layers "F.Cu" "B.Cu") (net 2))
 (segment (start 63.419999 62) (end 64.519999 62) (width 0.45) (layer "F.Cu") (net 4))
 (segment (start 55 62) (end 63.419999 62) (width 1.5) (layer "F.Cu") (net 4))
 (segment (start 65.48 62) (end 66.7125 62) (width 0.45) (layer "F.Cu") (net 6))
 (segment (start 70 60.98) (end 70 62) (width 0.45) (layer "F.Cu") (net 3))
 (segment (start 71.7125 62) (end 70 62) (width 0.45) (layer "F.Cu") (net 3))
 (segment (start 68.2875 62) (end 70 62) (width 0.45) (layer "F.Cu") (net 3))
 (segment (start 70 62.5125) (end 70 62) (width 0.45) (layer "F.Cu") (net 3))
 (segment (start 73.2875 62) (end 74.52 62) (width 0.45) (layer "F.Cu") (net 5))
 (segment (start 75.48 62) (end 76.58 62) (width 0.45) (layer "F.Cu") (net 1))
 (segment (start 76.58 62) (end 85 62) (width 1.5) (layer "F.Cu") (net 1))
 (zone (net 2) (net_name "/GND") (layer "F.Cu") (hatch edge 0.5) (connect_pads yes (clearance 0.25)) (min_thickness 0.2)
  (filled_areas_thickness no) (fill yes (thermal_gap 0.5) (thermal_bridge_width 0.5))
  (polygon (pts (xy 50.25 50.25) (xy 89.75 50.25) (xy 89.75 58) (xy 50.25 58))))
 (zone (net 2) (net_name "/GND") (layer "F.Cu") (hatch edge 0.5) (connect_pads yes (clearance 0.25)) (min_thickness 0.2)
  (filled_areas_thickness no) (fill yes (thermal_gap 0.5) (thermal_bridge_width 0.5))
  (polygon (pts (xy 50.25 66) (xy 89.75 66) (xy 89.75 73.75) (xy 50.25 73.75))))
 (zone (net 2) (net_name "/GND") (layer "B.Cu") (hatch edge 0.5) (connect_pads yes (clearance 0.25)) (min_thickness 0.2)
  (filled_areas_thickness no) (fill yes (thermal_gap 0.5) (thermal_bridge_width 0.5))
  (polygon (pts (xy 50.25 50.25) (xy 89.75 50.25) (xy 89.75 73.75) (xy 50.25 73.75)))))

